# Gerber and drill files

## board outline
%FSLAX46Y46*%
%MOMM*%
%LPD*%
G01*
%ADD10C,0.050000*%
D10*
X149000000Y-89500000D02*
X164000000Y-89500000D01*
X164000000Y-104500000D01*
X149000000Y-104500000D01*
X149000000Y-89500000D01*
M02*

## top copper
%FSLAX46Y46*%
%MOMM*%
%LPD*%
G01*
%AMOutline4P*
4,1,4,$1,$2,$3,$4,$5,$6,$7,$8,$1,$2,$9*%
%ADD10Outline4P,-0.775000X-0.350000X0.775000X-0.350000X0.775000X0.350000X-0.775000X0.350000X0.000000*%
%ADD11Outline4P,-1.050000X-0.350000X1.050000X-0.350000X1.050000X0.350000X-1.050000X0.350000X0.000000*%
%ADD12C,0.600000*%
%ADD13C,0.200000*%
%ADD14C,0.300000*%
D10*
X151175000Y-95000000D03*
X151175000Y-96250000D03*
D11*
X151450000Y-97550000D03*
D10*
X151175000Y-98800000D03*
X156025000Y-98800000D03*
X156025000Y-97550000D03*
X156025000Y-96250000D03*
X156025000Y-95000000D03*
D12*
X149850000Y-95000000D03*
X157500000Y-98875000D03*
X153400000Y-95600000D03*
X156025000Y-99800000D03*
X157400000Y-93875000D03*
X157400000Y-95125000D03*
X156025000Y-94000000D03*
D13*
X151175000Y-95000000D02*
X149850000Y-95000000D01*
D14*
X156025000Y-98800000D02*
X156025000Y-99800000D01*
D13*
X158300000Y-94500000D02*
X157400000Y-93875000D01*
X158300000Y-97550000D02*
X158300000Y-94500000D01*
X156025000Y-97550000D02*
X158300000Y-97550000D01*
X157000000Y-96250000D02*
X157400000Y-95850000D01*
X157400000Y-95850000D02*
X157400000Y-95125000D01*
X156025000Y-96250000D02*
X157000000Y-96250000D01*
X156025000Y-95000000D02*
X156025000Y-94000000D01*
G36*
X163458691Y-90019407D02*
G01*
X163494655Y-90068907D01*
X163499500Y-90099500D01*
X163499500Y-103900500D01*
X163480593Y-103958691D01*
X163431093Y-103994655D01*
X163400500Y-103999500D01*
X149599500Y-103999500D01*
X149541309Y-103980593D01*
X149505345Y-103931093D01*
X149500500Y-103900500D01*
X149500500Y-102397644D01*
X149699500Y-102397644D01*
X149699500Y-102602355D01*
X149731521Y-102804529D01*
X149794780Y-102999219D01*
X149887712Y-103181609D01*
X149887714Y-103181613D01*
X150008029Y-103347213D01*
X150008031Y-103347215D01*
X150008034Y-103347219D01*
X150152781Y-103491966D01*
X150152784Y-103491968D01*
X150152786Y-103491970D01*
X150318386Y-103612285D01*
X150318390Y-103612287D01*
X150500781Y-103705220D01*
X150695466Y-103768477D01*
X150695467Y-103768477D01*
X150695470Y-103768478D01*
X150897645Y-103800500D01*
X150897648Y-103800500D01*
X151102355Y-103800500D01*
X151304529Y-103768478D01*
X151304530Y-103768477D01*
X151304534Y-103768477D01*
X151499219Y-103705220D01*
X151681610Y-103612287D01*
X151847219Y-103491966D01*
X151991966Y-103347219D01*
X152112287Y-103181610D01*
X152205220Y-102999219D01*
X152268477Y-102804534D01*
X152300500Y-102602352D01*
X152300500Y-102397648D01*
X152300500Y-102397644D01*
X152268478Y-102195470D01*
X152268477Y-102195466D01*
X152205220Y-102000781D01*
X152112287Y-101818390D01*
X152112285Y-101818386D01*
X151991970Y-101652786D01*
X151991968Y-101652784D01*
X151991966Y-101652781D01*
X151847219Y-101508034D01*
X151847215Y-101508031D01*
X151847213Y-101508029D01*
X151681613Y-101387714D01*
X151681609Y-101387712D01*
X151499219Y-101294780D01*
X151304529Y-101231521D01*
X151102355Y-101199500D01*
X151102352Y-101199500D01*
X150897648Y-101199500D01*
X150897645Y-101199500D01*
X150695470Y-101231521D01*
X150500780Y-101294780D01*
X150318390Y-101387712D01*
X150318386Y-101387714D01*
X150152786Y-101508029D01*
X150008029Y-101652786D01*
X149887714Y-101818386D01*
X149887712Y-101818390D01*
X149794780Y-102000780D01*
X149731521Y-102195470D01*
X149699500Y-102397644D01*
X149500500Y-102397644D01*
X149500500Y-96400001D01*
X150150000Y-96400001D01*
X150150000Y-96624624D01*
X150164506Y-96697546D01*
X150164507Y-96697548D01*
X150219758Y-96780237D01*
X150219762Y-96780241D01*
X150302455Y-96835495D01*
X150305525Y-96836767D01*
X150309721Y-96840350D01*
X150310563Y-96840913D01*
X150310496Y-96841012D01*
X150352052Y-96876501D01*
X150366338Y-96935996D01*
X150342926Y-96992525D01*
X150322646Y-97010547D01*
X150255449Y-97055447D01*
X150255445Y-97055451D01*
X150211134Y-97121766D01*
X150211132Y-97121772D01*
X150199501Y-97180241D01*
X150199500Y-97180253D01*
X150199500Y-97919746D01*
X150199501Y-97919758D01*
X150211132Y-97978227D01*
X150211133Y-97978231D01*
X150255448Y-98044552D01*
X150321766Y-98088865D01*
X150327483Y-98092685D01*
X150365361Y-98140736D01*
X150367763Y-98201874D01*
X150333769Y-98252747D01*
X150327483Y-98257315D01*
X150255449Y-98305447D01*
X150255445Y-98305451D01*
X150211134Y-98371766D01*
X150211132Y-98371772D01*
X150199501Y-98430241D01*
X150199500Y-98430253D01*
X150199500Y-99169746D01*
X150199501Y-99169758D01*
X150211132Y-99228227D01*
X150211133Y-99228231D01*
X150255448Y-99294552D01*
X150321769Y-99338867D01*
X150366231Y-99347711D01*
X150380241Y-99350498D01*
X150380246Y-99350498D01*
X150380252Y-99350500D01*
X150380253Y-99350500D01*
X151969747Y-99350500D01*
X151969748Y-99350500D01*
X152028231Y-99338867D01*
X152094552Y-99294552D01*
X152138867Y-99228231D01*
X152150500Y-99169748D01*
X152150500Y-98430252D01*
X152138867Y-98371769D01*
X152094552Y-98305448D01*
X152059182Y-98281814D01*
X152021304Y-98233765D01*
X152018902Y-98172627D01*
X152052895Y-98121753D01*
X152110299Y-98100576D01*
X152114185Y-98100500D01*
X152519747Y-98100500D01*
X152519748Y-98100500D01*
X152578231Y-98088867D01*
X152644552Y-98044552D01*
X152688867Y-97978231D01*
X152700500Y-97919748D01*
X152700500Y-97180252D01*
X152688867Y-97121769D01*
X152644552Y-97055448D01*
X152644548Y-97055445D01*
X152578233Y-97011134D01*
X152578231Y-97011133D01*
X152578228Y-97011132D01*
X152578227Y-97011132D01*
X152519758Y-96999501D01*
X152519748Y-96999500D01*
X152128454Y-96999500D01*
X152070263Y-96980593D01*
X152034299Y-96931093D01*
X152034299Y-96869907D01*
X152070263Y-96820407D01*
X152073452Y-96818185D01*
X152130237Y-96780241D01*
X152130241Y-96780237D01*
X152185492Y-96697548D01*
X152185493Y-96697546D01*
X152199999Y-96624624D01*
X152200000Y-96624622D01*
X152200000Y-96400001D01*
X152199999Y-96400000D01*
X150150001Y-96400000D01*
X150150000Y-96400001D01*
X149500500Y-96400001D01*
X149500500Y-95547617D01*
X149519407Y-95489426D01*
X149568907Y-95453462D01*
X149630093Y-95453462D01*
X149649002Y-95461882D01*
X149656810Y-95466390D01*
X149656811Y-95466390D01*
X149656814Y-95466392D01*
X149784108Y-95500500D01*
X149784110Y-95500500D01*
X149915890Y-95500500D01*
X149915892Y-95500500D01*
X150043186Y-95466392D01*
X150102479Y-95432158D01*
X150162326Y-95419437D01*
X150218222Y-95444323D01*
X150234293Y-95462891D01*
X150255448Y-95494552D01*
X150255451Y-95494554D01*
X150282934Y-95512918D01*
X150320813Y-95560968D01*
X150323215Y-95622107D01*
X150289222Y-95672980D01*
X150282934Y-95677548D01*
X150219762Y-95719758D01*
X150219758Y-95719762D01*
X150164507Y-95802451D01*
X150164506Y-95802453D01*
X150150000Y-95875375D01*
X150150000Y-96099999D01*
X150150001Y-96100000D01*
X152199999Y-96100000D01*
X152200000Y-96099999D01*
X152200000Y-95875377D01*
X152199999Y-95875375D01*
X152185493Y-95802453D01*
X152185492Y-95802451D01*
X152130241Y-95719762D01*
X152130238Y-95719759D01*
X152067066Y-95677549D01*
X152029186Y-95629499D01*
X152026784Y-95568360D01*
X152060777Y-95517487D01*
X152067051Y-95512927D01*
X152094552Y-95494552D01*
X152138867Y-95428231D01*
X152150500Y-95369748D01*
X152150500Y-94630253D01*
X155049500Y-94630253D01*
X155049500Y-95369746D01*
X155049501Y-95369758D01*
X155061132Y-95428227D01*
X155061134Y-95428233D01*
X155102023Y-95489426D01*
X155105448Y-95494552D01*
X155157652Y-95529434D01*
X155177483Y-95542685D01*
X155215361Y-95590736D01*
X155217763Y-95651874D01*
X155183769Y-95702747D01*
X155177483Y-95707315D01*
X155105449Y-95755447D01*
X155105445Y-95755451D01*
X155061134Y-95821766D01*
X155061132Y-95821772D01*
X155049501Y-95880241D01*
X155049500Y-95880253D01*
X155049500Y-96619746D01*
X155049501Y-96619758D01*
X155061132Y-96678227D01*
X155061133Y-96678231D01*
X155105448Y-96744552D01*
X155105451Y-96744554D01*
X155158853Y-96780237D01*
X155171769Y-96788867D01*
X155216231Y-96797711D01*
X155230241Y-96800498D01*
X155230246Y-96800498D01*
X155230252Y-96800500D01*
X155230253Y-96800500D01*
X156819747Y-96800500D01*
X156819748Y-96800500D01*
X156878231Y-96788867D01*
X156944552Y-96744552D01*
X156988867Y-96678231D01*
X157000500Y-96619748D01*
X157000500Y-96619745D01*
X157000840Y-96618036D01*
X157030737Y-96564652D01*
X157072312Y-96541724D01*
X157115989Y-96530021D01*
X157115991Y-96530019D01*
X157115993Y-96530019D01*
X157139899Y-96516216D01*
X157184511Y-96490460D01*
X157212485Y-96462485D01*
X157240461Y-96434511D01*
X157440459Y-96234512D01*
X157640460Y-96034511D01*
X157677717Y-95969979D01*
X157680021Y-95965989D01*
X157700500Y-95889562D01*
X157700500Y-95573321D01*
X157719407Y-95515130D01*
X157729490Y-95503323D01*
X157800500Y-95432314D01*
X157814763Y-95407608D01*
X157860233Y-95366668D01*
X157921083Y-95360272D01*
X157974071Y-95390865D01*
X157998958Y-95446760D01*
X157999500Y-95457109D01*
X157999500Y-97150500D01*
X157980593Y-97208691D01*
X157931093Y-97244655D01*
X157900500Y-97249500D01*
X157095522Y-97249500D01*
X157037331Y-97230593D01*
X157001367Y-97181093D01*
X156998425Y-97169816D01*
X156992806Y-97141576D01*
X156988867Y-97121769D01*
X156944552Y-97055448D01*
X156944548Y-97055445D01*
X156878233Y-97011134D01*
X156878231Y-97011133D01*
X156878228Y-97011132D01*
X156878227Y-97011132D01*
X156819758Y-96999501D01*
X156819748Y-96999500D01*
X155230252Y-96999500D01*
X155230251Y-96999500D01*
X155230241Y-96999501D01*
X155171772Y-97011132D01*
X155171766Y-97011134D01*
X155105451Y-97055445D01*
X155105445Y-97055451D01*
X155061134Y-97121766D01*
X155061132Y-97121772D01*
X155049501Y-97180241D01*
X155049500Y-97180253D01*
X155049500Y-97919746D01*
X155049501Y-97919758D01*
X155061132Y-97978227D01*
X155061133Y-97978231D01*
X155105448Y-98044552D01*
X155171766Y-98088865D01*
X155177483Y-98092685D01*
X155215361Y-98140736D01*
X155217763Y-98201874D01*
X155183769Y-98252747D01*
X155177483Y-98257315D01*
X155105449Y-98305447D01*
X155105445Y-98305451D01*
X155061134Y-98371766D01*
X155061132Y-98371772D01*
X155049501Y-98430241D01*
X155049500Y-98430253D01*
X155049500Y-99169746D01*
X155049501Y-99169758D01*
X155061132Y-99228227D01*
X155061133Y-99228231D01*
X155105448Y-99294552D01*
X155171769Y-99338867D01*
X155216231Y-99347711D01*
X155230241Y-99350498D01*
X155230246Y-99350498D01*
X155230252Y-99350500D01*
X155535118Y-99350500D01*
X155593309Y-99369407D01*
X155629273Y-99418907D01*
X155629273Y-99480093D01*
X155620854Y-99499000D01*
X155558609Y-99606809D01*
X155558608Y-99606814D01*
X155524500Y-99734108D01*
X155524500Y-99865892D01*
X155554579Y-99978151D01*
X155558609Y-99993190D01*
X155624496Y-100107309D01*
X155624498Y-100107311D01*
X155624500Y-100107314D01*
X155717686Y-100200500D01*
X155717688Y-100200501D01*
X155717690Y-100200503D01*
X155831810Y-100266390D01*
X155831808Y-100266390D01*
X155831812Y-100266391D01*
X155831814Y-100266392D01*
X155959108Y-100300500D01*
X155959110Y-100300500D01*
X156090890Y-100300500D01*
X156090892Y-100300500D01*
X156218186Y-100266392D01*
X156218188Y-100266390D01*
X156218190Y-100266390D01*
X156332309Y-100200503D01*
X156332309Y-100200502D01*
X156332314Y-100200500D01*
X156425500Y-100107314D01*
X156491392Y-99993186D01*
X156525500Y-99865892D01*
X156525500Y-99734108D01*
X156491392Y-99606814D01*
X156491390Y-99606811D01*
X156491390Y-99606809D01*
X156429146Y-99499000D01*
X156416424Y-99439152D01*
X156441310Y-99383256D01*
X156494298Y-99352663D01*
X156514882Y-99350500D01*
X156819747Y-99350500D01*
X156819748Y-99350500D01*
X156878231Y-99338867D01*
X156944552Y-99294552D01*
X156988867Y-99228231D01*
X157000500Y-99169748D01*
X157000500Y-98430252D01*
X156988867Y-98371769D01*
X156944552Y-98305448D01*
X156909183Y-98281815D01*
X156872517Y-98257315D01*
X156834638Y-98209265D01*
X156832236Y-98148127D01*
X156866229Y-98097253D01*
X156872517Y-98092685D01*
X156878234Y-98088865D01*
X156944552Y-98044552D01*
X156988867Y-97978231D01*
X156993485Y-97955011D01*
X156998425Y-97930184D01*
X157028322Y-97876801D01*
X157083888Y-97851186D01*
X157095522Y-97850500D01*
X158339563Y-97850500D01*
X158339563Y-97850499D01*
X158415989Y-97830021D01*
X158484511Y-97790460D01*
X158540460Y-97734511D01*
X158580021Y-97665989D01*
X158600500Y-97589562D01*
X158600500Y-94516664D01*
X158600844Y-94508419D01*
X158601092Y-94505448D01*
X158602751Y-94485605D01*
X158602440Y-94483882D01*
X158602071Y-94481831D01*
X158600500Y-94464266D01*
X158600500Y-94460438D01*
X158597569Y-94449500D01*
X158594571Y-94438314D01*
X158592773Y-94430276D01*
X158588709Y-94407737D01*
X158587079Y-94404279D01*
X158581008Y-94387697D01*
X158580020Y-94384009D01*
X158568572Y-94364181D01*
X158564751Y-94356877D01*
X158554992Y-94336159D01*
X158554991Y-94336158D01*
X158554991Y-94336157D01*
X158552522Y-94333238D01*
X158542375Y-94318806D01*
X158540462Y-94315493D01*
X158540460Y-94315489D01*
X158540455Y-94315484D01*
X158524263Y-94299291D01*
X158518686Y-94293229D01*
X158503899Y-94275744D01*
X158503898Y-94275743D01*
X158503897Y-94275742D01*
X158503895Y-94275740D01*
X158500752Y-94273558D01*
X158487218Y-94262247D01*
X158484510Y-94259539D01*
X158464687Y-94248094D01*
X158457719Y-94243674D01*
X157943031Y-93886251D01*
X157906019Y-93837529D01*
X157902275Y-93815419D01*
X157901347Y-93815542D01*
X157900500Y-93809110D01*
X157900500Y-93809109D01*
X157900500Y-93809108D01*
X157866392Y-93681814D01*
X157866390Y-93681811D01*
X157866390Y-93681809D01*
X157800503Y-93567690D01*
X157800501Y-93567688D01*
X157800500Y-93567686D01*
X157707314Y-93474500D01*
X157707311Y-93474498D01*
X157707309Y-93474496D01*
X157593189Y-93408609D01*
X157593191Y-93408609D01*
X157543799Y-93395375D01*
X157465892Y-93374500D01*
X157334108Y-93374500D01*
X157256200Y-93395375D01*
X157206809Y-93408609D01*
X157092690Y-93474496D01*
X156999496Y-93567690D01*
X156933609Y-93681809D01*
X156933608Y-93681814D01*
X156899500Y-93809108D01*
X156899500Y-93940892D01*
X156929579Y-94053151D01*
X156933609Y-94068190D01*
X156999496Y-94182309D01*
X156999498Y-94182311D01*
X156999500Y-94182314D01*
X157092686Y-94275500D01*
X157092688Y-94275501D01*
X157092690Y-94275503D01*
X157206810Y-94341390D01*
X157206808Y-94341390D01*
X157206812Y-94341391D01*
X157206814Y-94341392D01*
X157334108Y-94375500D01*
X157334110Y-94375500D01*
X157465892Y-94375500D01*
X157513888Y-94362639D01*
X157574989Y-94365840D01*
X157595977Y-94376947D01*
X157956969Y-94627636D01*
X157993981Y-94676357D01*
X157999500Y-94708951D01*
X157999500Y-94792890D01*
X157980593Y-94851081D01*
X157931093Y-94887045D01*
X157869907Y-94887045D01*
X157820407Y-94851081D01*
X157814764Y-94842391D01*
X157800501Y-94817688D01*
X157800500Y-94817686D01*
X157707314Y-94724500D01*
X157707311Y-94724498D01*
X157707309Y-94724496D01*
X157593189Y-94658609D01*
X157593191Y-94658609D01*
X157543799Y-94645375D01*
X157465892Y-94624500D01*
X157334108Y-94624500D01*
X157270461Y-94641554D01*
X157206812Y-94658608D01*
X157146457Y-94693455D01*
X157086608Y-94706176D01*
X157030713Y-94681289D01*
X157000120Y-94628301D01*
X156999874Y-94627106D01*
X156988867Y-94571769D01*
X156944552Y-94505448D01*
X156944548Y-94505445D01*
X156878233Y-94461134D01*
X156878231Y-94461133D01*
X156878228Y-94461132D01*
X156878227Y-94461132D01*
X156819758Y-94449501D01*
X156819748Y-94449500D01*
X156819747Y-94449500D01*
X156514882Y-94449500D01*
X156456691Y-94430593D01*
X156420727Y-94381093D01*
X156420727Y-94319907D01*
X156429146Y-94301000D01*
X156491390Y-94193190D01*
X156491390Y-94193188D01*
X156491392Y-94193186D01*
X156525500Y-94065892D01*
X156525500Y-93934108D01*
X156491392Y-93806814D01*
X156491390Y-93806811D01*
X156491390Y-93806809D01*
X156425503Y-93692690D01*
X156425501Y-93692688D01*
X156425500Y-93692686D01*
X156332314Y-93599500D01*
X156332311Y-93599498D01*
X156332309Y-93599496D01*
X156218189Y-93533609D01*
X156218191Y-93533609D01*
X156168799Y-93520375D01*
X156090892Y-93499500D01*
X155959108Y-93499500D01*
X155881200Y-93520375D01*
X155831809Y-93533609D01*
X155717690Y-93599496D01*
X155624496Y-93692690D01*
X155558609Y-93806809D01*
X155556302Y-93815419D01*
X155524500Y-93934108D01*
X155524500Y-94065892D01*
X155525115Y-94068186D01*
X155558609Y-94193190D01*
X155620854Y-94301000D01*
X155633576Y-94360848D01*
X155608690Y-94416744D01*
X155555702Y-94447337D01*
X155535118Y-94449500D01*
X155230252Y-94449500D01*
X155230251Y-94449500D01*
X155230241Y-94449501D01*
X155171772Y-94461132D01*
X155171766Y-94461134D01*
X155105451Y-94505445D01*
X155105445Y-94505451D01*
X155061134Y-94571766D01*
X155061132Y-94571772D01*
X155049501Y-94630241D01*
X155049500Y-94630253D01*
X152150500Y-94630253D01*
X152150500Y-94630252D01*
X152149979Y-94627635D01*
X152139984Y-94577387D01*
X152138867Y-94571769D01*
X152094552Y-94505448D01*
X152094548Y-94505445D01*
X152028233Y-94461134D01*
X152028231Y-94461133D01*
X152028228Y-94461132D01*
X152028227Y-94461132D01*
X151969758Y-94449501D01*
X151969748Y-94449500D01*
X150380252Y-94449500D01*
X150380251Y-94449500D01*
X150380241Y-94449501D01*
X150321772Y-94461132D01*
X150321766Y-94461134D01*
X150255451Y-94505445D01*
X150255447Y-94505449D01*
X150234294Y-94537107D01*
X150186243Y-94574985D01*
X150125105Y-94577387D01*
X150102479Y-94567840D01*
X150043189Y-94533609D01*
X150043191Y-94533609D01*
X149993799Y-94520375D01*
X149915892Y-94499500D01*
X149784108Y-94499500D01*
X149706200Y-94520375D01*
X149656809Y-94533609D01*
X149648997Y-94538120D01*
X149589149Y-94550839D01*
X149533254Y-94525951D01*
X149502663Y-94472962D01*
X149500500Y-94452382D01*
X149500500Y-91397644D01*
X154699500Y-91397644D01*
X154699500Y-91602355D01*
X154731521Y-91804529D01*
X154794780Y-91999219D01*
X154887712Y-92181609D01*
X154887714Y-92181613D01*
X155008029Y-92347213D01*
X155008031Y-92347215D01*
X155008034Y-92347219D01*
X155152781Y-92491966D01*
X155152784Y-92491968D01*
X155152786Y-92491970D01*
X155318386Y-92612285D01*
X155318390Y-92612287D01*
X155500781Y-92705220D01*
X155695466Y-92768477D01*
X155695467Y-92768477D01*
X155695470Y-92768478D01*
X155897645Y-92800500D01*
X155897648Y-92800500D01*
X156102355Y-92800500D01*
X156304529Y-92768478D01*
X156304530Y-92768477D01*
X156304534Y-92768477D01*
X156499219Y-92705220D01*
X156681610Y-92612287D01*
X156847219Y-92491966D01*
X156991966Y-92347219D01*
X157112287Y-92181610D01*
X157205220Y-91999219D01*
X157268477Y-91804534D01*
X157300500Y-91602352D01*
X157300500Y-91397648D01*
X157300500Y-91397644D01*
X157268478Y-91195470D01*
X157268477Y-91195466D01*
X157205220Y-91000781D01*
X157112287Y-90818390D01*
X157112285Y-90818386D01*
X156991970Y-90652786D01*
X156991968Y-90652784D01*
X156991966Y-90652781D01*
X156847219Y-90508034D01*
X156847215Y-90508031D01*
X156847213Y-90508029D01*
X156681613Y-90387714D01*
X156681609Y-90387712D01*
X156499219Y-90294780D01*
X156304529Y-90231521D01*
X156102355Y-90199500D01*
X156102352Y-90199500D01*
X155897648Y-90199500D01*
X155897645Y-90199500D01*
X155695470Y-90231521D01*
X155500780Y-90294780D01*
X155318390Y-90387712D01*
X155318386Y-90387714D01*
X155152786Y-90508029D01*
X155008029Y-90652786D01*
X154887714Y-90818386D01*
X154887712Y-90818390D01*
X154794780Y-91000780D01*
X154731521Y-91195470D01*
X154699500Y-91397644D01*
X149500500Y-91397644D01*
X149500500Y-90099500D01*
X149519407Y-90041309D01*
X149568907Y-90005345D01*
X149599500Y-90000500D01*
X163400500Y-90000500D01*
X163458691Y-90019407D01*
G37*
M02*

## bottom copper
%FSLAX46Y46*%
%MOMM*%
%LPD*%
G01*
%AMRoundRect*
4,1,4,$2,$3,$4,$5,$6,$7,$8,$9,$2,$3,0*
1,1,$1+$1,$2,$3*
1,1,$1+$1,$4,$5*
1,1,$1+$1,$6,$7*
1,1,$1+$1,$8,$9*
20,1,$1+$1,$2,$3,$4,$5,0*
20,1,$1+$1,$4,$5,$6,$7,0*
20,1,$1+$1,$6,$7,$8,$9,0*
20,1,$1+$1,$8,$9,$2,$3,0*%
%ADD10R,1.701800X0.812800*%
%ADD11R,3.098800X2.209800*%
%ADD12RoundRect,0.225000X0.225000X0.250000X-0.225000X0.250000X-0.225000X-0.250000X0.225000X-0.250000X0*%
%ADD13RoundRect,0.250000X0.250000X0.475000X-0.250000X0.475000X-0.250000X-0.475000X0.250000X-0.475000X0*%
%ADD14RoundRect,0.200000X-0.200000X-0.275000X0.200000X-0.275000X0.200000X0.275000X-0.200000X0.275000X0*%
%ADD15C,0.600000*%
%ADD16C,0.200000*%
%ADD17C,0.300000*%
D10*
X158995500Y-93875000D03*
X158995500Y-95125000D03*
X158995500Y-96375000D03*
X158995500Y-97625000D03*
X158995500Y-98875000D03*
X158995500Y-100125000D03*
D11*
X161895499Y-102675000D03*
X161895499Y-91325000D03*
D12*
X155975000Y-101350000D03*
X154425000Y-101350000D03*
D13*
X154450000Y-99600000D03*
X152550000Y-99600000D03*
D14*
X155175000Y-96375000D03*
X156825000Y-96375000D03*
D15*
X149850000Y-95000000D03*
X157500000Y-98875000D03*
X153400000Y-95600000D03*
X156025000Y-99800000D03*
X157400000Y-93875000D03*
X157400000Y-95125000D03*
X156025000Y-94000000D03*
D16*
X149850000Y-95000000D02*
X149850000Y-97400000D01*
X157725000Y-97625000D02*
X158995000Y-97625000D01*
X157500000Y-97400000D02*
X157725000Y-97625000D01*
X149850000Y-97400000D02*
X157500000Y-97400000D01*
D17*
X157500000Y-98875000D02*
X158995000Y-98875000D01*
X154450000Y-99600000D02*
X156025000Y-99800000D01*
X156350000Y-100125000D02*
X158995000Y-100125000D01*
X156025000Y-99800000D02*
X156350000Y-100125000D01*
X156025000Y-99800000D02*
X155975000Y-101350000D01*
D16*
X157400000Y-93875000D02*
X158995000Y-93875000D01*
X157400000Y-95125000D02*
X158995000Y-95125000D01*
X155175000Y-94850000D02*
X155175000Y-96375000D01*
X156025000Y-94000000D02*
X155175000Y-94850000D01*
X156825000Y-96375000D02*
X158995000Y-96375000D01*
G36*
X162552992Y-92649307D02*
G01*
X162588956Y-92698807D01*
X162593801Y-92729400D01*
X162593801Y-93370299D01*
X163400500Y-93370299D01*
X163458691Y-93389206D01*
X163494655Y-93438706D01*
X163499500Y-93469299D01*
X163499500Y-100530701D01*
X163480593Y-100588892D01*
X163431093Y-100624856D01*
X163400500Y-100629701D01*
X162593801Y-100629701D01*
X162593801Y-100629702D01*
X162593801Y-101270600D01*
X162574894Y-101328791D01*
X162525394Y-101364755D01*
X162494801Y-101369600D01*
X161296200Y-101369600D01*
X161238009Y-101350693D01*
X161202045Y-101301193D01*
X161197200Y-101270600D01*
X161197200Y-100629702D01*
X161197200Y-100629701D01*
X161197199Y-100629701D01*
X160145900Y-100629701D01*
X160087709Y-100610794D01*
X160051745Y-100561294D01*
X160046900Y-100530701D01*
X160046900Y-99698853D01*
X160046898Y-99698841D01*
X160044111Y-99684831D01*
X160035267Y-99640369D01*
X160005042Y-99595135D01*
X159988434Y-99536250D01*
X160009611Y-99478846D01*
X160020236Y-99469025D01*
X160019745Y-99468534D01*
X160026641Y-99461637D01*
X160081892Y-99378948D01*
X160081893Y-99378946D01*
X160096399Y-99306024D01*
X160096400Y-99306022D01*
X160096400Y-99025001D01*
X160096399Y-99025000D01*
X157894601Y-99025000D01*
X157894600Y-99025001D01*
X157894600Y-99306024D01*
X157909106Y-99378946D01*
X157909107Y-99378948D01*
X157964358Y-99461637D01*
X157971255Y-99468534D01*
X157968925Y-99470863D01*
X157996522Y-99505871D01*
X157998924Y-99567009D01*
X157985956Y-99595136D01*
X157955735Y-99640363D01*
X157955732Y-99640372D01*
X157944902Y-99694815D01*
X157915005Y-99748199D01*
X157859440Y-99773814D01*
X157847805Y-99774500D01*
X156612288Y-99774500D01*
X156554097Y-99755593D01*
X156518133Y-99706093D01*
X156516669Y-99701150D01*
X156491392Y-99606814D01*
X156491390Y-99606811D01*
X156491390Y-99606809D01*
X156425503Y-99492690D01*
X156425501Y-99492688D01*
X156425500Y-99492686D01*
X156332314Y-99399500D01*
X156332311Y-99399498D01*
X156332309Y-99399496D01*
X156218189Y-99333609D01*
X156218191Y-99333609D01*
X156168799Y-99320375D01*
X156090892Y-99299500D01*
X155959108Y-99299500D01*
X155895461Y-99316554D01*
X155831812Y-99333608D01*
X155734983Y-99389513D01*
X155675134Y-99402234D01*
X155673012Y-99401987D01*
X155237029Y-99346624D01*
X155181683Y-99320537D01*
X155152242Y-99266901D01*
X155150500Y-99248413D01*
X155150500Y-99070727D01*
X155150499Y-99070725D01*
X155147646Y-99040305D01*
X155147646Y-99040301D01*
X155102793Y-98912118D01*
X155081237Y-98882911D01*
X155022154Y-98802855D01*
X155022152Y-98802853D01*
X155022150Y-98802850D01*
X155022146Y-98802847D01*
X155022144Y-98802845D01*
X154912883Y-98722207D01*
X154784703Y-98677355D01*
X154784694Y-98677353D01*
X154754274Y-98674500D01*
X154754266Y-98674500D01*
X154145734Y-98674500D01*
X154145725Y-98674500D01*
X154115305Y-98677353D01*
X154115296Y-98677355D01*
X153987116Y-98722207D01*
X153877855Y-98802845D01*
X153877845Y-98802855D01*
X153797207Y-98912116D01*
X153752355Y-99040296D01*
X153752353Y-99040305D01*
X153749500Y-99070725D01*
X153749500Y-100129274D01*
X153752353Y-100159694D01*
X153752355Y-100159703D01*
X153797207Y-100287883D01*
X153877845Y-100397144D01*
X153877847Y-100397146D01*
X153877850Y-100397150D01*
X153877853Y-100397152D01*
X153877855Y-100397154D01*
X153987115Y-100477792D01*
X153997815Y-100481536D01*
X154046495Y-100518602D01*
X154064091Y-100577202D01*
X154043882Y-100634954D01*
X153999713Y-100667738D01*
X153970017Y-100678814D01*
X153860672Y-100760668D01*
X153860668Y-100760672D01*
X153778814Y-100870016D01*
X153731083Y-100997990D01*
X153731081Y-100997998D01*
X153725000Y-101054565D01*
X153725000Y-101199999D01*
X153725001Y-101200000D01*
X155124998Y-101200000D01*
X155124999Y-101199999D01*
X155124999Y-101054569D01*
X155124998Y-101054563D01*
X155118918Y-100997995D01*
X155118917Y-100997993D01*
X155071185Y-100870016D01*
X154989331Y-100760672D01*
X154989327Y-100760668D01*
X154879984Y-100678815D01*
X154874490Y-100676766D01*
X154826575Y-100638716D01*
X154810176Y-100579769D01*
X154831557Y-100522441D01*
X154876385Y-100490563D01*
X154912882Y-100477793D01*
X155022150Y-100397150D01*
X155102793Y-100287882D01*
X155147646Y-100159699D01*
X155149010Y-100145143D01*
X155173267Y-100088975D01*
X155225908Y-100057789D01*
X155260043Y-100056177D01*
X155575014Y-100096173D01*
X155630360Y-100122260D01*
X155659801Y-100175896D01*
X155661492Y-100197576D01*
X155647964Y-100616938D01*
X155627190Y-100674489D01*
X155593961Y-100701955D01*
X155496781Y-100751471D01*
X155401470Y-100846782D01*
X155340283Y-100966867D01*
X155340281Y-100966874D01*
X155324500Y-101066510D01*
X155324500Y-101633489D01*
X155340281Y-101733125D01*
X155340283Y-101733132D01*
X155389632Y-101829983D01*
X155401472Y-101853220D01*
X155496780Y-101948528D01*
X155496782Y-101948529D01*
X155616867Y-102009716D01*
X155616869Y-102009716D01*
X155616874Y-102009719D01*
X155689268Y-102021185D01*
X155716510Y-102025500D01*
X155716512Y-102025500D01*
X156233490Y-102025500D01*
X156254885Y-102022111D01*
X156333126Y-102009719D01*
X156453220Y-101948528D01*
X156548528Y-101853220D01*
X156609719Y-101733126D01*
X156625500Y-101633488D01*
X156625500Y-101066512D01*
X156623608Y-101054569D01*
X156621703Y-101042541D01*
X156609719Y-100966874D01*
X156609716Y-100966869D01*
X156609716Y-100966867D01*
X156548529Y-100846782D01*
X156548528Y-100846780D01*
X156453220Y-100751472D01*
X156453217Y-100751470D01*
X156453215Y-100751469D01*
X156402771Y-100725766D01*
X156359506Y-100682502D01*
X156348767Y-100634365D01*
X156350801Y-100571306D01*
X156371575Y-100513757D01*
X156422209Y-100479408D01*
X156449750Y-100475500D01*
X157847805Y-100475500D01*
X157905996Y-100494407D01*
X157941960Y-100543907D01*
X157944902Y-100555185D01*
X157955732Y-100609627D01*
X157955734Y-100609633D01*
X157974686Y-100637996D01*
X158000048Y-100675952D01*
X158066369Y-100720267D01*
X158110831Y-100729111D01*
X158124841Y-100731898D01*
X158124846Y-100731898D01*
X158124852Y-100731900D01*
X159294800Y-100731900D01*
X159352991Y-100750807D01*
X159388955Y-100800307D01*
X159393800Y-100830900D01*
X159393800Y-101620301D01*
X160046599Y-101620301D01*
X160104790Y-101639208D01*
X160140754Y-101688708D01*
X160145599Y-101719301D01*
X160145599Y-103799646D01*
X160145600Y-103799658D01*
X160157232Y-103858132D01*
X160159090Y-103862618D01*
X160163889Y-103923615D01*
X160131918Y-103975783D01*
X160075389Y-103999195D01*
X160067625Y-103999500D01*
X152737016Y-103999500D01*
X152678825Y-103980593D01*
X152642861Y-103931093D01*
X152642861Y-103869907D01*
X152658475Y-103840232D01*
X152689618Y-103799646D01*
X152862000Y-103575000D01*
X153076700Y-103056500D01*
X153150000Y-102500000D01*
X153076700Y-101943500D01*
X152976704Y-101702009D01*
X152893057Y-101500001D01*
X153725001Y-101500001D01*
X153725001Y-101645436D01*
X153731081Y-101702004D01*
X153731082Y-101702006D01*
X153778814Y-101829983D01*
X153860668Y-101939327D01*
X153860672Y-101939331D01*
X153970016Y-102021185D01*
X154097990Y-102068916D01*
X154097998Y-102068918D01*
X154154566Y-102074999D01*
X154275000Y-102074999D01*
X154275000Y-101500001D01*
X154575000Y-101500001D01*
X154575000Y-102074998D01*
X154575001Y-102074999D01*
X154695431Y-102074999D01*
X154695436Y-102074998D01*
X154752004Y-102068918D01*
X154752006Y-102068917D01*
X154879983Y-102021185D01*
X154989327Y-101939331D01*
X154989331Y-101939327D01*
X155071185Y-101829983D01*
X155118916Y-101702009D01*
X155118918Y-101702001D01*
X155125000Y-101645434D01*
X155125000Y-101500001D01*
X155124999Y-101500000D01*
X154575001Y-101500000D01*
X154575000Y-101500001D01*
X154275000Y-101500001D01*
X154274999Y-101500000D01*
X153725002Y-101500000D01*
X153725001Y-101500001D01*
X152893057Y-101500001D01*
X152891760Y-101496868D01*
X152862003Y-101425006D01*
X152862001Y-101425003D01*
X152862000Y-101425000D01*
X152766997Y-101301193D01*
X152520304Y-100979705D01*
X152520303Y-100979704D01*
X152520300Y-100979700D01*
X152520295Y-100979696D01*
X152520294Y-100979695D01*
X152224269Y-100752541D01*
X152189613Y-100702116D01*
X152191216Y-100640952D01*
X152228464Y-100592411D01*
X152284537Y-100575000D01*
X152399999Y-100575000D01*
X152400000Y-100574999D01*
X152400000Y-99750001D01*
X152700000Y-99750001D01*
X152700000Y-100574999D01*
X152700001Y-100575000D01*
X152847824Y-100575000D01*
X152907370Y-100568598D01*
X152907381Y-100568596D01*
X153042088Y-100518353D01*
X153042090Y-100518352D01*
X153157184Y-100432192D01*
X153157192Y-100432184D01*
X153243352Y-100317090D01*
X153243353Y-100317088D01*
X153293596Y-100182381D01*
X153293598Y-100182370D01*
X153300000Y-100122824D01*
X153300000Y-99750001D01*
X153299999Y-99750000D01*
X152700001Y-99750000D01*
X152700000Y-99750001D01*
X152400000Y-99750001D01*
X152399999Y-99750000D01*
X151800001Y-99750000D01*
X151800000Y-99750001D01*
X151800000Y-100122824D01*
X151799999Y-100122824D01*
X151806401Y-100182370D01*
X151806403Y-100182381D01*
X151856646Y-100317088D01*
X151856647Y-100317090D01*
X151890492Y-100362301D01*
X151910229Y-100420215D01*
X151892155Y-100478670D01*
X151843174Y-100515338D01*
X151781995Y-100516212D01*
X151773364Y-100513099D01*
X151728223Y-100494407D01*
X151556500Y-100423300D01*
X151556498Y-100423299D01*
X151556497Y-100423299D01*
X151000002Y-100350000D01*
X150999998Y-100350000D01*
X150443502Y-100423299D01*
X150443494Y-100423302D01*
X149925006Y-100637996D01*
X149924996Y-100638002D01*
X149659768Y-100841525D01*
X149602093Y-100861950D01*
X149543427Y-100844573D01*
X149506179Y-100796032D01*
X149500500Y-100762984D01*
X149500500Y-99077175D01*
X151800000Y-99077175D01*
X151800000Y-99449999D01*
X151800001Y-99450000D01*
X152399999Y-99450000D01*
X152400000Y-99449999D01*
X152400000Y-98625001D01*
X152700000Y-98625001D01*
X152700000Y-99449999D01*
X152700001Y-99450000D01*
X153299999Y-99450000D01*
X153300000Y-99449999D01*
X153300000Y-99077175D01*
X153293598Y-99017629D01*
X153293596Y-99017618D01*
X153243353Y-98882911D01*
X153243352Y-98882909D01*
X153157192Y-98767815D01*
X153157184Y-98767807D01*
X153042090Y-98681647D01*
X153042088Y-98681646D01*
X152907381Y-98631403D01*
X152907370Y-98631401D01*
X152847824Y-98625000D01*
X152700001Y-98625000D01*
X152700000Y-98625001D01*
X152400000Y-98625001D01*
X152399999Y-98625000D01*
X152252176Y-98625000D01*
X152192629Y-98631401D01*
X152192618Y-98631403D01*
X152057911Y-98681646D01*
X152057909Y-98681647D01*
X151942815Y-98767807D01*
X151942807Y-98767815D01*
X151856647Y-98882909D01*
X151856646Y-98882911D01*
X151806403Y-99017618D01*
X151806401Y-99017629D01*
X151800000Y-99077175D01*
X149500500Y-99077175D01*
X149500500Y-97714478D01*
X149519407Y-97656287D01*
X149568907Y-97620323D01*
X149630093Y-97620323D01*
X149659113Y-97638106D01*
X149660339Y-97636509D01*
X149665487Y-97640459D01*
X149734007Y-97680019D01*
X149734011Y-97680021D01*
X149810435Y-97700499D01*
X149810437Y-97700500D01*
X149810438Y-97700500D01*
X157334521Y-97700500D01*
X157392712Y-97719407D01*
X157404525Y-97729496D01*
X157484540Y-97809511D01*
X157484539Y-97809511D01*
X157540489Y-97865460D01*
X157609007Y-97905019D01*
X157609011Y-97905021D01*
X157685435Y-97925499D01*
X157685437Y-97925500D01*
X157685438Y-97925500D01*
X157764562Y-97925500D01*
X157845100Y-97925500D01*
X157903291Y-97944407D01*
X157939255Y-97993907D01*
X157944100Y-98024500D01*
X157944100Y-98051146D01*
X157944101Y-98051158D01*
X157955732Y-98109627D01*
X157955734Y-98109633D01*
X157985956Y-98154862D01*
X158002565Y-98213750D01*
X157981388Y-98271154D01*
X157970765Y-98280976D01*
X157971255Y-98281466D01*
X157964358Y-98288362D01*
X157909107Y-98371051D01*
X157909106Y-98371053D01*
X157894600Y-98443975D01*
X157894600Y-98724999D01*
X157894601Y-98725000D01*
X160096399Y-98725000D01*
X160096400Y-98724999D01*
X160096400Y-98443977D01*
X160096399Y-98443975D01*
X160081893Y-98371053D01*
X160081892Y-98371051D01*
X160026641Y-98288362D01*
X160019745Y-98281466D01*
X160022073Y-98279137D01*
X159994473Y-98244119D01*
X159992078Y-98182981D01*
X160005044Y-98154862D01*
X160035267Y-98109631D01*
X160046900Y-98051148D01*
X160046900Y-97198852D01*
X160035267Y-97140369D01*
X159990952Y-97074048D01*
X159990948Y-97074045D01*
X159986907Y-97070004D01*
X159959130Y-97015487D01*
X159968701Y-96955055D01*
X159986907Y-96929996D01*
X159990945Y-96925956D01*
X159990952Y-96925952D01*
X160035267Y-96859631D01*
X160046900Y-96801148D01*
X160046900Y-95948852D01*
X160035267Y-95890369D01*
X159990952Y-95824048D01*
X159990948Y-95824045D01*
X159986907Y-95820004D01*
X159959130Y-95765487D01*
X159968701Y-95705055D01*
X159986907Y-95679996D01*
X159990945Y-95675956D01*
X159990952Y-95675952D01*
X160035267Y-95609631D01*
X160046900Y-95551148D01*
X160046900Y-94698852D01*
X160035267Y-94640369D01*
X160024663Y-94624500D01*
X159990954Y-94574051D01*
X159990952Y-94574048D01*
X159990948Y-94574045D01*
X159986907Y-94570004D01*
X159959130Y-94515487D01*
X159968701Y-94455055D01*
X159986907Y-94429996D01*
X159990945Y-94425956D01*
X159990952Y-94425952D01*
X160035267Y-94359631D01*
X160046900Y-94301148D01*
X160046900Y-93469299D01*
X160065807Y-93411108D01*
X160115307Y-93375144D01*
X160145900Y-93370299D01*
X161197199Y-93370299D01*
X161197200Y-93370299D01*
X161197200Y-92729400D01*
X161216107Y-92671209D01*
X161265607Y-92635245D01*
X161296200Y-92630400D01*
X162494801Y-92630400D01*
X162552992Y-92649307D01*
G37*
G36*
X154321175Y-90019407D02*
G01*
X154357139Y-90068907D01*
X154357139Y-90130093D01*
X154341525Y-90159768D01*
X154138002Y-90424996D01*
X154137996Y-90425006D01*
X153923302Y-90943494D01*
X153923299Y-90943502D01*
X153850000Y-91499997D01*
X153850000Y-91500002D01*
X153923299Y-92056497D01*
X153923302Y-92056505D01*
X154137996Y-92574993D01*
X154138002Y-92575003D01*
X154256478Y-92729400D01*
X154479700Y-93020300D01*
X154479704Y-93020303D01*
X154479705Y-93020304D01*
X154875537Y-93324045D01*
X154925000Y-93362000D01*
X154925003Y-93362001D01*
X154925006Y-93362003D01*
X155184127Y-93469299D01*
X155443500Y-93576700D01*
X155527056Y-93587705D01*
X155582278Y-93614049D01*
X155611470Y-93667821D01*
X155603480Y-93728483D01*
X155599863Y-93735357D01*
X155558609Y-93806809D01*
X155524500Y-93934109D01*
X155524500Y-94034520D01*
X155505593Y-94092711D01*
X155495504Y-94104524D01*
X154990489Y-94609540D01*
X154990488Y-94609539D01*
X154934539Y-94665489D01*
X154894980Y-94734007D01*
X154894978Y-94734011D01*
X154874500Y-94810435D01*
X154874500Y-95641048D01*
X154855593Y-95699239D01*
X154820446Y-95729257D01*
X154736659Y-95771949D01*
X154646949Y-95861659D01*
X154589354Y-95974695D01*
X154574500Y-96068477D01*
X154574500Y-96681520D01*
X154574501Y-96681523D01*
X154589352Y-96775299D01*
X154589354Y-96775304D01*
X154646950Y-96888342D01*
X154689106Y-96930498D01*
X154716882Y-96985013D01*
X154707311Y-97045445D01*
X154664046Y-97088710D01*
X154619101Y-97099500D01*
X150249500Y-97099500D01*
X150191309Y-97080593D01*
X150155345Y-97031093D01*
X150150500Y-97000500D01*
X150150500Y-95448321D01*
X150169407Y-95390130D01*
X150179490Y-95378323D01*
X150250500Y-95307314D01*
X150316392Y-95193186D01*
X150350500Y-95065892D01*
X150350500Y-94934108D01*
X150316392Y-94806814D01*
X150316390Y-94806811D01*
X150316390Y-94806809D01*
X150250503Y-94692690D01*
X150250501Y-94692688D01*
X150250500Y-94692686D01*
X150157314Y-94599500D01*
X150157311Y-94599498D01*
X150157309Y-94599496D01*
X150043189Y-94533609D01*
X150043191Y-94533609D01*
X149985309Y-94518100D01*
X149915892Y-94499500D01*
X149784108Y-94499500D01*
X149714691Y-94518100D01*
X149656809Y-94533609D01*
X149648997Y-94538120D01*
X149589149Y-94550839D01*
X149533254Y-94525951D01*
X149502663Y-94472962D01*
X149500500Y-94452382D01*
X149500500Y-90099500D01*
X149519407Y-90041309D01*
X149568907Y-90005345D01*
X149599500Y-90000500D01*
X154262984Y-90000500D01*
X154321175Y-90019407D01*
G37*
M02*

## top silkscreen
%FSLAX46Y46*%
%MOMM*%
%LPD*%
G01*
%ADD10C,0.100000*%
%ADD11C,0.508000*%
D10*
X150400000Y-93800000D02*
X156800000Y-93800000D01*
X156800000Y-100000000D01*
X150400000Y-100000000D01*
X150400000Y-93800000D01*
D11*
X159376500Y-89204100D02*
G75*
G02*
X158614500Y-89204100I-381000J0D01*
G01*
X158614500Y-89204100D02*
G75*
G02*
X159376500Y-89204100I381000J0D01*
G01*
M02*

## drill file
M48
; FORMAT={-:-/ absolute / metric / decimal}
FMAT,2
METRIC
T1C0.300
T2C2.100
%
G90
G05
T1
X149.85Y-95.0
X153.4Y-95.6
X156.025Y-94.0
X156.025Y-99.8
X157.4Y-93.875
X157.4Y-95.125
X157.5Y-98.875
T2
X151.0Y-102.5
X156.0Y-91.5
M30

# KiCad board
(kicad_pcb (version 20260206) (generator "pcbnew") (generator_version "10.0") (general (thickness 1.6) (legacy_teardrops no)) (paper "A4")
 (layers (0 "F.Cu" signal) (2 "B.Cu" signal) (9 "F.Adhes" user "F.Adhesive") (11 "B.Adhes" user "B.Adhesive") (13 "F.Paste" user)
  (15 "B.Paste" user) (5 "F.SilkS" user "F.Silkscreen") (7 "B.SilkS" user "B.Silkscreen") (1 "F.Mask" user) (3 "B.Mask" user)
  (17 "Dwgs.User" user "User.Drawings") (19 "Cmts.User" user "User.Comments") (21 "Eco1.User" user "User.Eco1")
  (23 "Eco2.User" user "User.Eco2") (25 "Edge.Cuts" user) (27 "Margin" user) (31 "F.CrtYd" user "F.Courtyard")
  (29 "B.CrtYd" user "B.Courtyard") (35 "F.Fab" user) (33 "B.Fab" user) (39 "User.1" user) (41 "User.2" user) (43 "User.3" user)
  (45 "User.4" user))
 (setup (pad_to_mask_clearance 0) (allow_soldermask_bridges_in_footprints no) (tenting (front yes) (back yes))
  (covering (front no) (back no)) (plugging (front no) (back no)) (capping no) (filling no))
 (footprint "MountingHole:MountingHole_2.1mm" (layer "F.Cu") (at 151 102.5)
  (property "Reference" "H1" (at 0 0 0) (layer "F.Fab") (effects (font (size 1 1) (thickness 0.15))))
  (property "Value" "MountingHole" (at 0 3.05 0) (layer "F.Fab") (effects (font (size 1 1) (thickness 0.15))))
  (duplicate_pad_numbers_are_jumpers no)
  (pad "" np_thru_hole circle (at 0 0) (size 2.1 2.1) (drill 2.1) (layers "*.Cu" "*.Mask")))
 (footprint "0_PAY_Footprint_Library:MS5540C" (layer "F.Cu") (at 150.4 100)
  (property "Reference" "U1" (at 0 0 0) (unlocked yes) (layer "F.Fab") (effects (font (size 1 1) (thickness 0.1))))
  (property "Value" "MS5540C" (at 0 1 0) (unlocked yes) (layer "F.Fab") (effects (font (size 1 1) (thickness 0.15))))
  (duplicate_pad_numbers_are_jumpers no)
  (fp_rect (start 0 0) (end 6.4 -6.2) (stroke (width 0.1) (type solid)) (fill no) (layer "F.SilkS"))
  (pad "1" smd trapezoid (at 0.775 -5) (size 1.55 0.7) (layers "F.Cu" "F.Mask" "F.Paste") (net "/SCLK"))
  (pad "2" smd trapezoid (at 0.775 -3.75) (size 1.55 0.7) (layers "F.Cu" "F.Mask" "F.Paste") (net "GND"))
  (pad "3" smd trapezoid (at 1.05 -2.45) (size 2.1 0.7) (layers "F.Cu" "F.Mask" "F.Paste") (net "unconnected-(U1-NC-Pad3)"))
  (pad "4" smd trapezoid (at 0.775 -1.2) (size 1.55 0.7) (layers "F.Cu" "F.Mask" "F.Paste") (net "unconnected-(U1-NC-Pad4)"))
  (pad "5" smd trapezoid (at 5.625 -1.2) (size 1.55 0.7) (layers "F.Cu" "F.Mask" "F.Paste") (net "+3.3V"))
  (pad "6" smd trapezoid (at 5.625 -2.45) (size 1.55 0.7) (layers "F.Cu" "F.Mask" "F.Paste") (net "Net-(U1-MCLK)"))
  (pad "7" smd trapezoid (at 5.625 -3.75) (size 1.55 0.7) (layers "F.Cu" "F.Mask" "F.Paste") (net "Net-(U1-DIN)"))
  (pad "8" smd trapezoid (at 5.625 -5) (size 1.55 0.7) (layers "F.Cu" "F.Mask" "F.Paste") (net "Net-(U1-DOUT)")))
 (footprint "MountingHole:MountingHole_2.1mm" (layer "F.Cu") (at 156 91.5)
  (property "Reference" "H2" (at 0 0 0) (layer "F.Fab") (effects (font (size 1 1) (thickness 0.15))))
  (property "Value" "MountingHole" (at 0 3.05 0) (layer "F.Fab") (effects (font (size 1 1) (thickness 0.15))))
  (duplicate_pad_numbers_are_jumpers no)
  (pad "" np_thru_hole circle (at 0 0) (size 2.1 2.1) (drill 2.1) (layers "*.Cu" "*.Mask")))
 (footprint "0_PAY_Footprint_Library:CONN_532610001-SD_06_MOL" (layer "B.Cu") (at 161.9 97 90)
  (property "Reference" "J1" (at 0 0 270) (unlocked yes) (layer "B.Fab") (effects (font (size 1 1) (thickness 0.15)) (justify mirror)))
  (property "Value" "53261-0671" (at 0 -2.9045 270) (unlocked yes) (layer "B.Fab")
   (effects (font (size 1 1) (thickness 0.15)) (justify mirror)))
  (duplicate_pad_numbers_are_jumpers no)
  (fp_circle (center 7.7959 -2.9045) (end 8.1769 -2.9045) (stroke (width 0.508) (type solid)) (fill no) (layer "F.SilkS"))
  (pad "1" smd rect (at 3.125 -2.9045 90) (size 0.8128 1.7018) (layers "B.Cu" "B.Mask" "B.Paste") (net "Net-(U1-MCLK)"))
  (pad "2" smd rect (at 1.875 -2.9045 90) (size 0.8128 1.7018) (layers "B.Cu" "B.Mask" "B.Paste") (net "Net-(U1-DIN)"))
  (pad "3" smd rect (at 0.625 -2.9045 90) (size 0.8128 1.7018) (layers "B.Cu" "B.Mask" "B.Paste") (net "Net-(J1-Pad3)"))
  (pad "4" smd rect (at -0.625 -2.9045 90) (size 0.8128 1.7018) (layers "B.Cu" "B.Mask" "B.Paste") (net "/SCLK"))
  (pad "5" smd rect (at -1.875 -2.9045 90) (size 0.8128 1.7018) (layers "B.Cu" "B.Mask" "B.Paste") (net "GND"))
  (pad "6" smd rect (at -3.125 -2.9045 90) (size 0.8128 1.7018) (layers "B.Cu" "B.Mask" "B.Paste") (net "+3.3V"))
  (pad "7" smd rect (at -5.675 -0.004501 90) (size 2.2098 3.0988) (layers "B.Cu" "B.Mask" "B.Paste"))
  (pad "8" smd rect (at 5.675 -0.004501 90) (size 2.2098 3.0988) (layers "B.Cu" "B.Mask" "B.Paste"))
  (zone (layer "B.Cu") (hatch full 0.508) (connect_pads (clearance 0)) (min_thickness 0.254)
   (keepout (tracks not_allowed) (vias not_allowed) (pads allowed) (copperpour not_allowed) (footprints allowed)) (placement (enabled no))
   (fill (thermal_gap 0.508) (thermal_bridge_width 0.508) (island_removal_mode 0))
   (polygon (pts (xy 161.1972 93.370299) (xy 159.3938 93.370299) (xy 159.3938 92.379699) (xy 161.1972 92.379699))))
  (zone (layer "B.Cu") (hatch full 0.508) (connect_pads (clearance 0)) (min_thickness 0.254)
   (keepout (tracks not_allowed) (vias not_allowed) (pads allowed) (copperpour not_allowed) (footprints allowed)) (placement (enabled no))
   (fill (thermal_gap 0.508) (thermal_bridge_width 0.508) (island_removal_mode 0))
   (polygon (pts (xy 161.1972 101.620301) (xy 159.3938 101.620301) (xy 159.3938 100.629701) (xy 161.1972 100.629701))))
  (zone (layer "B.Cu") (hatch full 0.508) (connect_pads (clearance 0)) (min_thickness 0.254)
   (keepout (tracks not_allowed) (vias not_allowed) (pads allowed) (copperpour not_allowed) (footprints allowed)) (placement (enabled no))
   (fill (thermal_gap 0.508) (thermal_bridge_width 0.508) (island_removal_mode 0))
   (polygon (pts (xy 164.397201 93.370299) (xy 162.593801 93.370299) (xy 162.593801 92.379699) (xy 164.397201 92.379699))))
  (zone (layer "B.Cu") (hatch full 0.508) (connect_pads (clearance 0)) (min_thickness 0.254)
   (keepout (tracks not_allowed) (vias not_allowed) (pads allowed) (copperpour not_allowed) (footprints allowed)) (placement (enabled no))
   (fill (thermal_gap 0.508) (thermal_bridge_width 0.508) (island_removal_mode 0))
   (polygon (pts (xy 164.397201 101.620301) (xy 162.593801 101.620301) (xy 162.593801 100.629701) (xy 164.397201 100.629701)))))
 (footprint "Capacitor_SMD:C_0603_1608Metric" (layer "B.Cu") (at 155.2 101.35 180)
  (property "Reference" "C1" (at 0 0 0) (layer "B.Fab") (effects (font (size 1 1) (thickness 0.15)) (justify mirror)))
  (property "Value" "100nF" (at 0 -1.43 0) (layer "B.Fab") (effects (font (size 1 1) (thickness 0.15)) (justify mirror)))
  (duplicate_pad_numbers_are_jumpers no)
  (pad "1" smd roundrect (at -0.775 0 180) (size 0.9 0.95) (layers "B.Cu" "B.Mask" "B.Paste") (roundrect_rratio 0.25) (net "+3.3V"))
  (pad "2" smd roundrect (at 0.775 0 180) (size 0.9 0.95) (layers "B.Cu" "B.Mask" "B.Paste") (roundrect_rratio 0.25) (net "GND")))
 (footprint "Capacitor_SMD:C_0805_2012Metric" (layer "B.Cu") (at 153.5 99.6 180)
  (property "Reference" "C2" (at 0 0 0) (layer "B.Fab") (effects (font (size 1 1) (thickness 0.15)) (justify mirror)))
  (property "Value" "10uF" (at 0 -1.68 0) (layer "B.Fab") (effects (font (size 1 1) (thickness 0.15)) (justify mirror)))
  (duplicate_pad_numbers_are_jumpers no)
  (pad "1" smd roundrect (at -0.95 0 180) (size 1 1.45) (layers "B.Cu" "B.Mask" "B.Paste") (roundrect_rratio 0.25) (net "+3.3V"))
  (pad "2" smd roundrect (at 0.95 0 180) (size 1 1.45) (layers "B.Cu" "B.Mask" "B.Paste") (roundrect_rratio 0.25) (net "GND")))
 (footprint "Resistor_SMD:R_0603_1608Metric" (layer "B.Cu") (at 156 96.375)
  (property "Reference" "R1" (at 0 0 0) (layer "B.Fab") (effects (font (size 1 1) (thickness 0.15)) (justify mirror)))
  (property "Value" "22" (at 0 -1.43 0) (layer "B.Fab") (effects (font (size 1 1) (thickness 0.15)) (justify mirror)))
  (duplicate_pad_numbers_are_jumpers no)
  (pad "1" smd roundrect (at -0.825 0) (size 0.8 0.95) (layers "B.Cu" "B.Mask" "B.Paste") (roundrect_rratio 0.25) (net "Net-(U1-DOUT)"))
  (pad "2" smd roundrect (at 0.825 0) (size 0.8 0.95) (layers "B.Cu" "B.Mask" "B.Paste") (roundrect_rratio 0.25) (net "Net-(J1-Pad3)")))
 (gr_rect (start 149 89.5) (end 164 104.5) (stroke (width 0.05) (type default)) (fill no) (layer "Edge.Cuts"))
 (segment (start 151.175 95) (end 149.85 95) (width 0.2) (layer "F.Cu") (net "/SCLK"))
 (via (at 149.85 95) (size 0.6) (drill 0.3) (layers "F.Cu" "B.Cu") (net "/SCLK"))
 (segment (start 149.85 95) (end 149.85 97.4) (width 0.2) (layer "B.Cu") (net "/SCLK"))
 (segment (start 157.725 97.625) (end 158.995 97.625) (width 0.2) (layer "B.Cu") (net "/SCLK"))
 (segment (start 157.5 97.4) (end 157.725 97.625) (width 0.2) (layer "B.Cu") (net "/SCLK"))
 (segment (start 149.85 97.4) (end 157.5 97.4) (width 0.2) (layer "B.Cu") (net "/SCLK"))
 (via (at 157.5 98.875) (size 0.6) (drill 0.3) (layers "F.Cu" "B.Cu") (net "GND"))
 (via (at 153.4 95.6) (size 0.6) (drill 0.3) (layers "F.Cu" "B.Cu") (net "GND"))
 (segment (start 157.5 98.875) (end 158.995 98.875) (width 0.3) (layer "B.Cu") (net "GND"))
 (segment (start 156.025 98.8) (end 156.025 99.8) (width 0.3) (layer "F.Cu") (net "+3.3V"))
 (via (at 156.025 99.8) (size 0.6) (drill 0.3) (layers "F.Cu" "B.Cu") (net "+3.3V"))
 (segment (start 154.45 99.6) (end 156.025 99.8) (width 0.3) (layer "B.Cu") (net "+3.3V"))
 (segment (start 156.35 100.125) (end 158.995 100.125) (width 0.3) (layer "B.Cu") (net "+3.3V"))
 (segment (start 156.025 99.8) (end 156.35 100.125) (width 0.3) (layer "B.Cu") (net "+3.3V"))
 (segment (start 156.025 99.8) (end 155.975 101.35) (width 0.3) (layer "B.Cu") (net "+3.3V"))
 (segment (start 158.3 94.5) (end 157.4 93.875) (width 0.2) (layer "F.Cu") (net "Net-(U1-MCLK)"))
 (segment (start 158.3 97.55) (end 158.3 94.5) (width 0.2) (layer "F.Cu") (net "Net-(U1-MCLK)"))
 (segment (start 156.025 97.55) (end 158.3 97.55) (width 0.2) (layer "F.Cu") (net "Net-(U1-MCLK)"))
 (via (at 157.4 93.875) (size 0.6) (drill 0.3) (layers "F.Cu" "B.Cu") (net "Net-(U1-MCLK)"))
 (segment (start 157.4 93.875) (end 158.995 93.875) (width 0.2) (layer "B.Cu") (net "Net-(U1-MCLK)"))
 (segment (start 157 96.25) (end 157.4 95.85) (width 0.2) (layer "F.Cu") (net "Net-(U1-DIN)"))
 (segment (start 157.4 95.85) (end 157.4 95.125) (width 0.2) (layer "F.Cu") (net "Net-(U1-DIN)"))
 (segment (start 156.025 96.25) (end 157 96.25) (width 0.2) (layer "F.Cu") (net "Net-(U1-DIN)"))
 (via (at 157.4 95.125) (size 0.6) (drill 0.3) (layers "F.Cu" "B.Cu") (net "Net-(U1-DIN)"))
 (segment (start 157.4 95.125) (end 158.995 95.125) (width 0.2) (layer "B.Cu") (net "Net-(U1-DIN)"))
 (segment (start 156.025 95) (end 156.025 94) (width 0.2) (layer "F.Cu") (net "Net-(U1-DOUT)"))
 (via (at 156.025 94) (size 0.6) (drill 0.3) (layers "F.Cu" "B.Cu") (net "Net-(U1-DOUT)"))
 (segment (start 155.175 94.85) (end 155.175 96.375) (width 0.2) (layer "B.Cu") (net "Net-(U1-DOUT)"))
 (segment (start 156.025 94) (end 155.175 94.85) (width 0.2) (layer "B.Cu") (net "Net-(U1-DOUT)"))
 (segment (start 156.825 96.375) (end 158.995 96.375) (width 0.2) (layer "B.Cu") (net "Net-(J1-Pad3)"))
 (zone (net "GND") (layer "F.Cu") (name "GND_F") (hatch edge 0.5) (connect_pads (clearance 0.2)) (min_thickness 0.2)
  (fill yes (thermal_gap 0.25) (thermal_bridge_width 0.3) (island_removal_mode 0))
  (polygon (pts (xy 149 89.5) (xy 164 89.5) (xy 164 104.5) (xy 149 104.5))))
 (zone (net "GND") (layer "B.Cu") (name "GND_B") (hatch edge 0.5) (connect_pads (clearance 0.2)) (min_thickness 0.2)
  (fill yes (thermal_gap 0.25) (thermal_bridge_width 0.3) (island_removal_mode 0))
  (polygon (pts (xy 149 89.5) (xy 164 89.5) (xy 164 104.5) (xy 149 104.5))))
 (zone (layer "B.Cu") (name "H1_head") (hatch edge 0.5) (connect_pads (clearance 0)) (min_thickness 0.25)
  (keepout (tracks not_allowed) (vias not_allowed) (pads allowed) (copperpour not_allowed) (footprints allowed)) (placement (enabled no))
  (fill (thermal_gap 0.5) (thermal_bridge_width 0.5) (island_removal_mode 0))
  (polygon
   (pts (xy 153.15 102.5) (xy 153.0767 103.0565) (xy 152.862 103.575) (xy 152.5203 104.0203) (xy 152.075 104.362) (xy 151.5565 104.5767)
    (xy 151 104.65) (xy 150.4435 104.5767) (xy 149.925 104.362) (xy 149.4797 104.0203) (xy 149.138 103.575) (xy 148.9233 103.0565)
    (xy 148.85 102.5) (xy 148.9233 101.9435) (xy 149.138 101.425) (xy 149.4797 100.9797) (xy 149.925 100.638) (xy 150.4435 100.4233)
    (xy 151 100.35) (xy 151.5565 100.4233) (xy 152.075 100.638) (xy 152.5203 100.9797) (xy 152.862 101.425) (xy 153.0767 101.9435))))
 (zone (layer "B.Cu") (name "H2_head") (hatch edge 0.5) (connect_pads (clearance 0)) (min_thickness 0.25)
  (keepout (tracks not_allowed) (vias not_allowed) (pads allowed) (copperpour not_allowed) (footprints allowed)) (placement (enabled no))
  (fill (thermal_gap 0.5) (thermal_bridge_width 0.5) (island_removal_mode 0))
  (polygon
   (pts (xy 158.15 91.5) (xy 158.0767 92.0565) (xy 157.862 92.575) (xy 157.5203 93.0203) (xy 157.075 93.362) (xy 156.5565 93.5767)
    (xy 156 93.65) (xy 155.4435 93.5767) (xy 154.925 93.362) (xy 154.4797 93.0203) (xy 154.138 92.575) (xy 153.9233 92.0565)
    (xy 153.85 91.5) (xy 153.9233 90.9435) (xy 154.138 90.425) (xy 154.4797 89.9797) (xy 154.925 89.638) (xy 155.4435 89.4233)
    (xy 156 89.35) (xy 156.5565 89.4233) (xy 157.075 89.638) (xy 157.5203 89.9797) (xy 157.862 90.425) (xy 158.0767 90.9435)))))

